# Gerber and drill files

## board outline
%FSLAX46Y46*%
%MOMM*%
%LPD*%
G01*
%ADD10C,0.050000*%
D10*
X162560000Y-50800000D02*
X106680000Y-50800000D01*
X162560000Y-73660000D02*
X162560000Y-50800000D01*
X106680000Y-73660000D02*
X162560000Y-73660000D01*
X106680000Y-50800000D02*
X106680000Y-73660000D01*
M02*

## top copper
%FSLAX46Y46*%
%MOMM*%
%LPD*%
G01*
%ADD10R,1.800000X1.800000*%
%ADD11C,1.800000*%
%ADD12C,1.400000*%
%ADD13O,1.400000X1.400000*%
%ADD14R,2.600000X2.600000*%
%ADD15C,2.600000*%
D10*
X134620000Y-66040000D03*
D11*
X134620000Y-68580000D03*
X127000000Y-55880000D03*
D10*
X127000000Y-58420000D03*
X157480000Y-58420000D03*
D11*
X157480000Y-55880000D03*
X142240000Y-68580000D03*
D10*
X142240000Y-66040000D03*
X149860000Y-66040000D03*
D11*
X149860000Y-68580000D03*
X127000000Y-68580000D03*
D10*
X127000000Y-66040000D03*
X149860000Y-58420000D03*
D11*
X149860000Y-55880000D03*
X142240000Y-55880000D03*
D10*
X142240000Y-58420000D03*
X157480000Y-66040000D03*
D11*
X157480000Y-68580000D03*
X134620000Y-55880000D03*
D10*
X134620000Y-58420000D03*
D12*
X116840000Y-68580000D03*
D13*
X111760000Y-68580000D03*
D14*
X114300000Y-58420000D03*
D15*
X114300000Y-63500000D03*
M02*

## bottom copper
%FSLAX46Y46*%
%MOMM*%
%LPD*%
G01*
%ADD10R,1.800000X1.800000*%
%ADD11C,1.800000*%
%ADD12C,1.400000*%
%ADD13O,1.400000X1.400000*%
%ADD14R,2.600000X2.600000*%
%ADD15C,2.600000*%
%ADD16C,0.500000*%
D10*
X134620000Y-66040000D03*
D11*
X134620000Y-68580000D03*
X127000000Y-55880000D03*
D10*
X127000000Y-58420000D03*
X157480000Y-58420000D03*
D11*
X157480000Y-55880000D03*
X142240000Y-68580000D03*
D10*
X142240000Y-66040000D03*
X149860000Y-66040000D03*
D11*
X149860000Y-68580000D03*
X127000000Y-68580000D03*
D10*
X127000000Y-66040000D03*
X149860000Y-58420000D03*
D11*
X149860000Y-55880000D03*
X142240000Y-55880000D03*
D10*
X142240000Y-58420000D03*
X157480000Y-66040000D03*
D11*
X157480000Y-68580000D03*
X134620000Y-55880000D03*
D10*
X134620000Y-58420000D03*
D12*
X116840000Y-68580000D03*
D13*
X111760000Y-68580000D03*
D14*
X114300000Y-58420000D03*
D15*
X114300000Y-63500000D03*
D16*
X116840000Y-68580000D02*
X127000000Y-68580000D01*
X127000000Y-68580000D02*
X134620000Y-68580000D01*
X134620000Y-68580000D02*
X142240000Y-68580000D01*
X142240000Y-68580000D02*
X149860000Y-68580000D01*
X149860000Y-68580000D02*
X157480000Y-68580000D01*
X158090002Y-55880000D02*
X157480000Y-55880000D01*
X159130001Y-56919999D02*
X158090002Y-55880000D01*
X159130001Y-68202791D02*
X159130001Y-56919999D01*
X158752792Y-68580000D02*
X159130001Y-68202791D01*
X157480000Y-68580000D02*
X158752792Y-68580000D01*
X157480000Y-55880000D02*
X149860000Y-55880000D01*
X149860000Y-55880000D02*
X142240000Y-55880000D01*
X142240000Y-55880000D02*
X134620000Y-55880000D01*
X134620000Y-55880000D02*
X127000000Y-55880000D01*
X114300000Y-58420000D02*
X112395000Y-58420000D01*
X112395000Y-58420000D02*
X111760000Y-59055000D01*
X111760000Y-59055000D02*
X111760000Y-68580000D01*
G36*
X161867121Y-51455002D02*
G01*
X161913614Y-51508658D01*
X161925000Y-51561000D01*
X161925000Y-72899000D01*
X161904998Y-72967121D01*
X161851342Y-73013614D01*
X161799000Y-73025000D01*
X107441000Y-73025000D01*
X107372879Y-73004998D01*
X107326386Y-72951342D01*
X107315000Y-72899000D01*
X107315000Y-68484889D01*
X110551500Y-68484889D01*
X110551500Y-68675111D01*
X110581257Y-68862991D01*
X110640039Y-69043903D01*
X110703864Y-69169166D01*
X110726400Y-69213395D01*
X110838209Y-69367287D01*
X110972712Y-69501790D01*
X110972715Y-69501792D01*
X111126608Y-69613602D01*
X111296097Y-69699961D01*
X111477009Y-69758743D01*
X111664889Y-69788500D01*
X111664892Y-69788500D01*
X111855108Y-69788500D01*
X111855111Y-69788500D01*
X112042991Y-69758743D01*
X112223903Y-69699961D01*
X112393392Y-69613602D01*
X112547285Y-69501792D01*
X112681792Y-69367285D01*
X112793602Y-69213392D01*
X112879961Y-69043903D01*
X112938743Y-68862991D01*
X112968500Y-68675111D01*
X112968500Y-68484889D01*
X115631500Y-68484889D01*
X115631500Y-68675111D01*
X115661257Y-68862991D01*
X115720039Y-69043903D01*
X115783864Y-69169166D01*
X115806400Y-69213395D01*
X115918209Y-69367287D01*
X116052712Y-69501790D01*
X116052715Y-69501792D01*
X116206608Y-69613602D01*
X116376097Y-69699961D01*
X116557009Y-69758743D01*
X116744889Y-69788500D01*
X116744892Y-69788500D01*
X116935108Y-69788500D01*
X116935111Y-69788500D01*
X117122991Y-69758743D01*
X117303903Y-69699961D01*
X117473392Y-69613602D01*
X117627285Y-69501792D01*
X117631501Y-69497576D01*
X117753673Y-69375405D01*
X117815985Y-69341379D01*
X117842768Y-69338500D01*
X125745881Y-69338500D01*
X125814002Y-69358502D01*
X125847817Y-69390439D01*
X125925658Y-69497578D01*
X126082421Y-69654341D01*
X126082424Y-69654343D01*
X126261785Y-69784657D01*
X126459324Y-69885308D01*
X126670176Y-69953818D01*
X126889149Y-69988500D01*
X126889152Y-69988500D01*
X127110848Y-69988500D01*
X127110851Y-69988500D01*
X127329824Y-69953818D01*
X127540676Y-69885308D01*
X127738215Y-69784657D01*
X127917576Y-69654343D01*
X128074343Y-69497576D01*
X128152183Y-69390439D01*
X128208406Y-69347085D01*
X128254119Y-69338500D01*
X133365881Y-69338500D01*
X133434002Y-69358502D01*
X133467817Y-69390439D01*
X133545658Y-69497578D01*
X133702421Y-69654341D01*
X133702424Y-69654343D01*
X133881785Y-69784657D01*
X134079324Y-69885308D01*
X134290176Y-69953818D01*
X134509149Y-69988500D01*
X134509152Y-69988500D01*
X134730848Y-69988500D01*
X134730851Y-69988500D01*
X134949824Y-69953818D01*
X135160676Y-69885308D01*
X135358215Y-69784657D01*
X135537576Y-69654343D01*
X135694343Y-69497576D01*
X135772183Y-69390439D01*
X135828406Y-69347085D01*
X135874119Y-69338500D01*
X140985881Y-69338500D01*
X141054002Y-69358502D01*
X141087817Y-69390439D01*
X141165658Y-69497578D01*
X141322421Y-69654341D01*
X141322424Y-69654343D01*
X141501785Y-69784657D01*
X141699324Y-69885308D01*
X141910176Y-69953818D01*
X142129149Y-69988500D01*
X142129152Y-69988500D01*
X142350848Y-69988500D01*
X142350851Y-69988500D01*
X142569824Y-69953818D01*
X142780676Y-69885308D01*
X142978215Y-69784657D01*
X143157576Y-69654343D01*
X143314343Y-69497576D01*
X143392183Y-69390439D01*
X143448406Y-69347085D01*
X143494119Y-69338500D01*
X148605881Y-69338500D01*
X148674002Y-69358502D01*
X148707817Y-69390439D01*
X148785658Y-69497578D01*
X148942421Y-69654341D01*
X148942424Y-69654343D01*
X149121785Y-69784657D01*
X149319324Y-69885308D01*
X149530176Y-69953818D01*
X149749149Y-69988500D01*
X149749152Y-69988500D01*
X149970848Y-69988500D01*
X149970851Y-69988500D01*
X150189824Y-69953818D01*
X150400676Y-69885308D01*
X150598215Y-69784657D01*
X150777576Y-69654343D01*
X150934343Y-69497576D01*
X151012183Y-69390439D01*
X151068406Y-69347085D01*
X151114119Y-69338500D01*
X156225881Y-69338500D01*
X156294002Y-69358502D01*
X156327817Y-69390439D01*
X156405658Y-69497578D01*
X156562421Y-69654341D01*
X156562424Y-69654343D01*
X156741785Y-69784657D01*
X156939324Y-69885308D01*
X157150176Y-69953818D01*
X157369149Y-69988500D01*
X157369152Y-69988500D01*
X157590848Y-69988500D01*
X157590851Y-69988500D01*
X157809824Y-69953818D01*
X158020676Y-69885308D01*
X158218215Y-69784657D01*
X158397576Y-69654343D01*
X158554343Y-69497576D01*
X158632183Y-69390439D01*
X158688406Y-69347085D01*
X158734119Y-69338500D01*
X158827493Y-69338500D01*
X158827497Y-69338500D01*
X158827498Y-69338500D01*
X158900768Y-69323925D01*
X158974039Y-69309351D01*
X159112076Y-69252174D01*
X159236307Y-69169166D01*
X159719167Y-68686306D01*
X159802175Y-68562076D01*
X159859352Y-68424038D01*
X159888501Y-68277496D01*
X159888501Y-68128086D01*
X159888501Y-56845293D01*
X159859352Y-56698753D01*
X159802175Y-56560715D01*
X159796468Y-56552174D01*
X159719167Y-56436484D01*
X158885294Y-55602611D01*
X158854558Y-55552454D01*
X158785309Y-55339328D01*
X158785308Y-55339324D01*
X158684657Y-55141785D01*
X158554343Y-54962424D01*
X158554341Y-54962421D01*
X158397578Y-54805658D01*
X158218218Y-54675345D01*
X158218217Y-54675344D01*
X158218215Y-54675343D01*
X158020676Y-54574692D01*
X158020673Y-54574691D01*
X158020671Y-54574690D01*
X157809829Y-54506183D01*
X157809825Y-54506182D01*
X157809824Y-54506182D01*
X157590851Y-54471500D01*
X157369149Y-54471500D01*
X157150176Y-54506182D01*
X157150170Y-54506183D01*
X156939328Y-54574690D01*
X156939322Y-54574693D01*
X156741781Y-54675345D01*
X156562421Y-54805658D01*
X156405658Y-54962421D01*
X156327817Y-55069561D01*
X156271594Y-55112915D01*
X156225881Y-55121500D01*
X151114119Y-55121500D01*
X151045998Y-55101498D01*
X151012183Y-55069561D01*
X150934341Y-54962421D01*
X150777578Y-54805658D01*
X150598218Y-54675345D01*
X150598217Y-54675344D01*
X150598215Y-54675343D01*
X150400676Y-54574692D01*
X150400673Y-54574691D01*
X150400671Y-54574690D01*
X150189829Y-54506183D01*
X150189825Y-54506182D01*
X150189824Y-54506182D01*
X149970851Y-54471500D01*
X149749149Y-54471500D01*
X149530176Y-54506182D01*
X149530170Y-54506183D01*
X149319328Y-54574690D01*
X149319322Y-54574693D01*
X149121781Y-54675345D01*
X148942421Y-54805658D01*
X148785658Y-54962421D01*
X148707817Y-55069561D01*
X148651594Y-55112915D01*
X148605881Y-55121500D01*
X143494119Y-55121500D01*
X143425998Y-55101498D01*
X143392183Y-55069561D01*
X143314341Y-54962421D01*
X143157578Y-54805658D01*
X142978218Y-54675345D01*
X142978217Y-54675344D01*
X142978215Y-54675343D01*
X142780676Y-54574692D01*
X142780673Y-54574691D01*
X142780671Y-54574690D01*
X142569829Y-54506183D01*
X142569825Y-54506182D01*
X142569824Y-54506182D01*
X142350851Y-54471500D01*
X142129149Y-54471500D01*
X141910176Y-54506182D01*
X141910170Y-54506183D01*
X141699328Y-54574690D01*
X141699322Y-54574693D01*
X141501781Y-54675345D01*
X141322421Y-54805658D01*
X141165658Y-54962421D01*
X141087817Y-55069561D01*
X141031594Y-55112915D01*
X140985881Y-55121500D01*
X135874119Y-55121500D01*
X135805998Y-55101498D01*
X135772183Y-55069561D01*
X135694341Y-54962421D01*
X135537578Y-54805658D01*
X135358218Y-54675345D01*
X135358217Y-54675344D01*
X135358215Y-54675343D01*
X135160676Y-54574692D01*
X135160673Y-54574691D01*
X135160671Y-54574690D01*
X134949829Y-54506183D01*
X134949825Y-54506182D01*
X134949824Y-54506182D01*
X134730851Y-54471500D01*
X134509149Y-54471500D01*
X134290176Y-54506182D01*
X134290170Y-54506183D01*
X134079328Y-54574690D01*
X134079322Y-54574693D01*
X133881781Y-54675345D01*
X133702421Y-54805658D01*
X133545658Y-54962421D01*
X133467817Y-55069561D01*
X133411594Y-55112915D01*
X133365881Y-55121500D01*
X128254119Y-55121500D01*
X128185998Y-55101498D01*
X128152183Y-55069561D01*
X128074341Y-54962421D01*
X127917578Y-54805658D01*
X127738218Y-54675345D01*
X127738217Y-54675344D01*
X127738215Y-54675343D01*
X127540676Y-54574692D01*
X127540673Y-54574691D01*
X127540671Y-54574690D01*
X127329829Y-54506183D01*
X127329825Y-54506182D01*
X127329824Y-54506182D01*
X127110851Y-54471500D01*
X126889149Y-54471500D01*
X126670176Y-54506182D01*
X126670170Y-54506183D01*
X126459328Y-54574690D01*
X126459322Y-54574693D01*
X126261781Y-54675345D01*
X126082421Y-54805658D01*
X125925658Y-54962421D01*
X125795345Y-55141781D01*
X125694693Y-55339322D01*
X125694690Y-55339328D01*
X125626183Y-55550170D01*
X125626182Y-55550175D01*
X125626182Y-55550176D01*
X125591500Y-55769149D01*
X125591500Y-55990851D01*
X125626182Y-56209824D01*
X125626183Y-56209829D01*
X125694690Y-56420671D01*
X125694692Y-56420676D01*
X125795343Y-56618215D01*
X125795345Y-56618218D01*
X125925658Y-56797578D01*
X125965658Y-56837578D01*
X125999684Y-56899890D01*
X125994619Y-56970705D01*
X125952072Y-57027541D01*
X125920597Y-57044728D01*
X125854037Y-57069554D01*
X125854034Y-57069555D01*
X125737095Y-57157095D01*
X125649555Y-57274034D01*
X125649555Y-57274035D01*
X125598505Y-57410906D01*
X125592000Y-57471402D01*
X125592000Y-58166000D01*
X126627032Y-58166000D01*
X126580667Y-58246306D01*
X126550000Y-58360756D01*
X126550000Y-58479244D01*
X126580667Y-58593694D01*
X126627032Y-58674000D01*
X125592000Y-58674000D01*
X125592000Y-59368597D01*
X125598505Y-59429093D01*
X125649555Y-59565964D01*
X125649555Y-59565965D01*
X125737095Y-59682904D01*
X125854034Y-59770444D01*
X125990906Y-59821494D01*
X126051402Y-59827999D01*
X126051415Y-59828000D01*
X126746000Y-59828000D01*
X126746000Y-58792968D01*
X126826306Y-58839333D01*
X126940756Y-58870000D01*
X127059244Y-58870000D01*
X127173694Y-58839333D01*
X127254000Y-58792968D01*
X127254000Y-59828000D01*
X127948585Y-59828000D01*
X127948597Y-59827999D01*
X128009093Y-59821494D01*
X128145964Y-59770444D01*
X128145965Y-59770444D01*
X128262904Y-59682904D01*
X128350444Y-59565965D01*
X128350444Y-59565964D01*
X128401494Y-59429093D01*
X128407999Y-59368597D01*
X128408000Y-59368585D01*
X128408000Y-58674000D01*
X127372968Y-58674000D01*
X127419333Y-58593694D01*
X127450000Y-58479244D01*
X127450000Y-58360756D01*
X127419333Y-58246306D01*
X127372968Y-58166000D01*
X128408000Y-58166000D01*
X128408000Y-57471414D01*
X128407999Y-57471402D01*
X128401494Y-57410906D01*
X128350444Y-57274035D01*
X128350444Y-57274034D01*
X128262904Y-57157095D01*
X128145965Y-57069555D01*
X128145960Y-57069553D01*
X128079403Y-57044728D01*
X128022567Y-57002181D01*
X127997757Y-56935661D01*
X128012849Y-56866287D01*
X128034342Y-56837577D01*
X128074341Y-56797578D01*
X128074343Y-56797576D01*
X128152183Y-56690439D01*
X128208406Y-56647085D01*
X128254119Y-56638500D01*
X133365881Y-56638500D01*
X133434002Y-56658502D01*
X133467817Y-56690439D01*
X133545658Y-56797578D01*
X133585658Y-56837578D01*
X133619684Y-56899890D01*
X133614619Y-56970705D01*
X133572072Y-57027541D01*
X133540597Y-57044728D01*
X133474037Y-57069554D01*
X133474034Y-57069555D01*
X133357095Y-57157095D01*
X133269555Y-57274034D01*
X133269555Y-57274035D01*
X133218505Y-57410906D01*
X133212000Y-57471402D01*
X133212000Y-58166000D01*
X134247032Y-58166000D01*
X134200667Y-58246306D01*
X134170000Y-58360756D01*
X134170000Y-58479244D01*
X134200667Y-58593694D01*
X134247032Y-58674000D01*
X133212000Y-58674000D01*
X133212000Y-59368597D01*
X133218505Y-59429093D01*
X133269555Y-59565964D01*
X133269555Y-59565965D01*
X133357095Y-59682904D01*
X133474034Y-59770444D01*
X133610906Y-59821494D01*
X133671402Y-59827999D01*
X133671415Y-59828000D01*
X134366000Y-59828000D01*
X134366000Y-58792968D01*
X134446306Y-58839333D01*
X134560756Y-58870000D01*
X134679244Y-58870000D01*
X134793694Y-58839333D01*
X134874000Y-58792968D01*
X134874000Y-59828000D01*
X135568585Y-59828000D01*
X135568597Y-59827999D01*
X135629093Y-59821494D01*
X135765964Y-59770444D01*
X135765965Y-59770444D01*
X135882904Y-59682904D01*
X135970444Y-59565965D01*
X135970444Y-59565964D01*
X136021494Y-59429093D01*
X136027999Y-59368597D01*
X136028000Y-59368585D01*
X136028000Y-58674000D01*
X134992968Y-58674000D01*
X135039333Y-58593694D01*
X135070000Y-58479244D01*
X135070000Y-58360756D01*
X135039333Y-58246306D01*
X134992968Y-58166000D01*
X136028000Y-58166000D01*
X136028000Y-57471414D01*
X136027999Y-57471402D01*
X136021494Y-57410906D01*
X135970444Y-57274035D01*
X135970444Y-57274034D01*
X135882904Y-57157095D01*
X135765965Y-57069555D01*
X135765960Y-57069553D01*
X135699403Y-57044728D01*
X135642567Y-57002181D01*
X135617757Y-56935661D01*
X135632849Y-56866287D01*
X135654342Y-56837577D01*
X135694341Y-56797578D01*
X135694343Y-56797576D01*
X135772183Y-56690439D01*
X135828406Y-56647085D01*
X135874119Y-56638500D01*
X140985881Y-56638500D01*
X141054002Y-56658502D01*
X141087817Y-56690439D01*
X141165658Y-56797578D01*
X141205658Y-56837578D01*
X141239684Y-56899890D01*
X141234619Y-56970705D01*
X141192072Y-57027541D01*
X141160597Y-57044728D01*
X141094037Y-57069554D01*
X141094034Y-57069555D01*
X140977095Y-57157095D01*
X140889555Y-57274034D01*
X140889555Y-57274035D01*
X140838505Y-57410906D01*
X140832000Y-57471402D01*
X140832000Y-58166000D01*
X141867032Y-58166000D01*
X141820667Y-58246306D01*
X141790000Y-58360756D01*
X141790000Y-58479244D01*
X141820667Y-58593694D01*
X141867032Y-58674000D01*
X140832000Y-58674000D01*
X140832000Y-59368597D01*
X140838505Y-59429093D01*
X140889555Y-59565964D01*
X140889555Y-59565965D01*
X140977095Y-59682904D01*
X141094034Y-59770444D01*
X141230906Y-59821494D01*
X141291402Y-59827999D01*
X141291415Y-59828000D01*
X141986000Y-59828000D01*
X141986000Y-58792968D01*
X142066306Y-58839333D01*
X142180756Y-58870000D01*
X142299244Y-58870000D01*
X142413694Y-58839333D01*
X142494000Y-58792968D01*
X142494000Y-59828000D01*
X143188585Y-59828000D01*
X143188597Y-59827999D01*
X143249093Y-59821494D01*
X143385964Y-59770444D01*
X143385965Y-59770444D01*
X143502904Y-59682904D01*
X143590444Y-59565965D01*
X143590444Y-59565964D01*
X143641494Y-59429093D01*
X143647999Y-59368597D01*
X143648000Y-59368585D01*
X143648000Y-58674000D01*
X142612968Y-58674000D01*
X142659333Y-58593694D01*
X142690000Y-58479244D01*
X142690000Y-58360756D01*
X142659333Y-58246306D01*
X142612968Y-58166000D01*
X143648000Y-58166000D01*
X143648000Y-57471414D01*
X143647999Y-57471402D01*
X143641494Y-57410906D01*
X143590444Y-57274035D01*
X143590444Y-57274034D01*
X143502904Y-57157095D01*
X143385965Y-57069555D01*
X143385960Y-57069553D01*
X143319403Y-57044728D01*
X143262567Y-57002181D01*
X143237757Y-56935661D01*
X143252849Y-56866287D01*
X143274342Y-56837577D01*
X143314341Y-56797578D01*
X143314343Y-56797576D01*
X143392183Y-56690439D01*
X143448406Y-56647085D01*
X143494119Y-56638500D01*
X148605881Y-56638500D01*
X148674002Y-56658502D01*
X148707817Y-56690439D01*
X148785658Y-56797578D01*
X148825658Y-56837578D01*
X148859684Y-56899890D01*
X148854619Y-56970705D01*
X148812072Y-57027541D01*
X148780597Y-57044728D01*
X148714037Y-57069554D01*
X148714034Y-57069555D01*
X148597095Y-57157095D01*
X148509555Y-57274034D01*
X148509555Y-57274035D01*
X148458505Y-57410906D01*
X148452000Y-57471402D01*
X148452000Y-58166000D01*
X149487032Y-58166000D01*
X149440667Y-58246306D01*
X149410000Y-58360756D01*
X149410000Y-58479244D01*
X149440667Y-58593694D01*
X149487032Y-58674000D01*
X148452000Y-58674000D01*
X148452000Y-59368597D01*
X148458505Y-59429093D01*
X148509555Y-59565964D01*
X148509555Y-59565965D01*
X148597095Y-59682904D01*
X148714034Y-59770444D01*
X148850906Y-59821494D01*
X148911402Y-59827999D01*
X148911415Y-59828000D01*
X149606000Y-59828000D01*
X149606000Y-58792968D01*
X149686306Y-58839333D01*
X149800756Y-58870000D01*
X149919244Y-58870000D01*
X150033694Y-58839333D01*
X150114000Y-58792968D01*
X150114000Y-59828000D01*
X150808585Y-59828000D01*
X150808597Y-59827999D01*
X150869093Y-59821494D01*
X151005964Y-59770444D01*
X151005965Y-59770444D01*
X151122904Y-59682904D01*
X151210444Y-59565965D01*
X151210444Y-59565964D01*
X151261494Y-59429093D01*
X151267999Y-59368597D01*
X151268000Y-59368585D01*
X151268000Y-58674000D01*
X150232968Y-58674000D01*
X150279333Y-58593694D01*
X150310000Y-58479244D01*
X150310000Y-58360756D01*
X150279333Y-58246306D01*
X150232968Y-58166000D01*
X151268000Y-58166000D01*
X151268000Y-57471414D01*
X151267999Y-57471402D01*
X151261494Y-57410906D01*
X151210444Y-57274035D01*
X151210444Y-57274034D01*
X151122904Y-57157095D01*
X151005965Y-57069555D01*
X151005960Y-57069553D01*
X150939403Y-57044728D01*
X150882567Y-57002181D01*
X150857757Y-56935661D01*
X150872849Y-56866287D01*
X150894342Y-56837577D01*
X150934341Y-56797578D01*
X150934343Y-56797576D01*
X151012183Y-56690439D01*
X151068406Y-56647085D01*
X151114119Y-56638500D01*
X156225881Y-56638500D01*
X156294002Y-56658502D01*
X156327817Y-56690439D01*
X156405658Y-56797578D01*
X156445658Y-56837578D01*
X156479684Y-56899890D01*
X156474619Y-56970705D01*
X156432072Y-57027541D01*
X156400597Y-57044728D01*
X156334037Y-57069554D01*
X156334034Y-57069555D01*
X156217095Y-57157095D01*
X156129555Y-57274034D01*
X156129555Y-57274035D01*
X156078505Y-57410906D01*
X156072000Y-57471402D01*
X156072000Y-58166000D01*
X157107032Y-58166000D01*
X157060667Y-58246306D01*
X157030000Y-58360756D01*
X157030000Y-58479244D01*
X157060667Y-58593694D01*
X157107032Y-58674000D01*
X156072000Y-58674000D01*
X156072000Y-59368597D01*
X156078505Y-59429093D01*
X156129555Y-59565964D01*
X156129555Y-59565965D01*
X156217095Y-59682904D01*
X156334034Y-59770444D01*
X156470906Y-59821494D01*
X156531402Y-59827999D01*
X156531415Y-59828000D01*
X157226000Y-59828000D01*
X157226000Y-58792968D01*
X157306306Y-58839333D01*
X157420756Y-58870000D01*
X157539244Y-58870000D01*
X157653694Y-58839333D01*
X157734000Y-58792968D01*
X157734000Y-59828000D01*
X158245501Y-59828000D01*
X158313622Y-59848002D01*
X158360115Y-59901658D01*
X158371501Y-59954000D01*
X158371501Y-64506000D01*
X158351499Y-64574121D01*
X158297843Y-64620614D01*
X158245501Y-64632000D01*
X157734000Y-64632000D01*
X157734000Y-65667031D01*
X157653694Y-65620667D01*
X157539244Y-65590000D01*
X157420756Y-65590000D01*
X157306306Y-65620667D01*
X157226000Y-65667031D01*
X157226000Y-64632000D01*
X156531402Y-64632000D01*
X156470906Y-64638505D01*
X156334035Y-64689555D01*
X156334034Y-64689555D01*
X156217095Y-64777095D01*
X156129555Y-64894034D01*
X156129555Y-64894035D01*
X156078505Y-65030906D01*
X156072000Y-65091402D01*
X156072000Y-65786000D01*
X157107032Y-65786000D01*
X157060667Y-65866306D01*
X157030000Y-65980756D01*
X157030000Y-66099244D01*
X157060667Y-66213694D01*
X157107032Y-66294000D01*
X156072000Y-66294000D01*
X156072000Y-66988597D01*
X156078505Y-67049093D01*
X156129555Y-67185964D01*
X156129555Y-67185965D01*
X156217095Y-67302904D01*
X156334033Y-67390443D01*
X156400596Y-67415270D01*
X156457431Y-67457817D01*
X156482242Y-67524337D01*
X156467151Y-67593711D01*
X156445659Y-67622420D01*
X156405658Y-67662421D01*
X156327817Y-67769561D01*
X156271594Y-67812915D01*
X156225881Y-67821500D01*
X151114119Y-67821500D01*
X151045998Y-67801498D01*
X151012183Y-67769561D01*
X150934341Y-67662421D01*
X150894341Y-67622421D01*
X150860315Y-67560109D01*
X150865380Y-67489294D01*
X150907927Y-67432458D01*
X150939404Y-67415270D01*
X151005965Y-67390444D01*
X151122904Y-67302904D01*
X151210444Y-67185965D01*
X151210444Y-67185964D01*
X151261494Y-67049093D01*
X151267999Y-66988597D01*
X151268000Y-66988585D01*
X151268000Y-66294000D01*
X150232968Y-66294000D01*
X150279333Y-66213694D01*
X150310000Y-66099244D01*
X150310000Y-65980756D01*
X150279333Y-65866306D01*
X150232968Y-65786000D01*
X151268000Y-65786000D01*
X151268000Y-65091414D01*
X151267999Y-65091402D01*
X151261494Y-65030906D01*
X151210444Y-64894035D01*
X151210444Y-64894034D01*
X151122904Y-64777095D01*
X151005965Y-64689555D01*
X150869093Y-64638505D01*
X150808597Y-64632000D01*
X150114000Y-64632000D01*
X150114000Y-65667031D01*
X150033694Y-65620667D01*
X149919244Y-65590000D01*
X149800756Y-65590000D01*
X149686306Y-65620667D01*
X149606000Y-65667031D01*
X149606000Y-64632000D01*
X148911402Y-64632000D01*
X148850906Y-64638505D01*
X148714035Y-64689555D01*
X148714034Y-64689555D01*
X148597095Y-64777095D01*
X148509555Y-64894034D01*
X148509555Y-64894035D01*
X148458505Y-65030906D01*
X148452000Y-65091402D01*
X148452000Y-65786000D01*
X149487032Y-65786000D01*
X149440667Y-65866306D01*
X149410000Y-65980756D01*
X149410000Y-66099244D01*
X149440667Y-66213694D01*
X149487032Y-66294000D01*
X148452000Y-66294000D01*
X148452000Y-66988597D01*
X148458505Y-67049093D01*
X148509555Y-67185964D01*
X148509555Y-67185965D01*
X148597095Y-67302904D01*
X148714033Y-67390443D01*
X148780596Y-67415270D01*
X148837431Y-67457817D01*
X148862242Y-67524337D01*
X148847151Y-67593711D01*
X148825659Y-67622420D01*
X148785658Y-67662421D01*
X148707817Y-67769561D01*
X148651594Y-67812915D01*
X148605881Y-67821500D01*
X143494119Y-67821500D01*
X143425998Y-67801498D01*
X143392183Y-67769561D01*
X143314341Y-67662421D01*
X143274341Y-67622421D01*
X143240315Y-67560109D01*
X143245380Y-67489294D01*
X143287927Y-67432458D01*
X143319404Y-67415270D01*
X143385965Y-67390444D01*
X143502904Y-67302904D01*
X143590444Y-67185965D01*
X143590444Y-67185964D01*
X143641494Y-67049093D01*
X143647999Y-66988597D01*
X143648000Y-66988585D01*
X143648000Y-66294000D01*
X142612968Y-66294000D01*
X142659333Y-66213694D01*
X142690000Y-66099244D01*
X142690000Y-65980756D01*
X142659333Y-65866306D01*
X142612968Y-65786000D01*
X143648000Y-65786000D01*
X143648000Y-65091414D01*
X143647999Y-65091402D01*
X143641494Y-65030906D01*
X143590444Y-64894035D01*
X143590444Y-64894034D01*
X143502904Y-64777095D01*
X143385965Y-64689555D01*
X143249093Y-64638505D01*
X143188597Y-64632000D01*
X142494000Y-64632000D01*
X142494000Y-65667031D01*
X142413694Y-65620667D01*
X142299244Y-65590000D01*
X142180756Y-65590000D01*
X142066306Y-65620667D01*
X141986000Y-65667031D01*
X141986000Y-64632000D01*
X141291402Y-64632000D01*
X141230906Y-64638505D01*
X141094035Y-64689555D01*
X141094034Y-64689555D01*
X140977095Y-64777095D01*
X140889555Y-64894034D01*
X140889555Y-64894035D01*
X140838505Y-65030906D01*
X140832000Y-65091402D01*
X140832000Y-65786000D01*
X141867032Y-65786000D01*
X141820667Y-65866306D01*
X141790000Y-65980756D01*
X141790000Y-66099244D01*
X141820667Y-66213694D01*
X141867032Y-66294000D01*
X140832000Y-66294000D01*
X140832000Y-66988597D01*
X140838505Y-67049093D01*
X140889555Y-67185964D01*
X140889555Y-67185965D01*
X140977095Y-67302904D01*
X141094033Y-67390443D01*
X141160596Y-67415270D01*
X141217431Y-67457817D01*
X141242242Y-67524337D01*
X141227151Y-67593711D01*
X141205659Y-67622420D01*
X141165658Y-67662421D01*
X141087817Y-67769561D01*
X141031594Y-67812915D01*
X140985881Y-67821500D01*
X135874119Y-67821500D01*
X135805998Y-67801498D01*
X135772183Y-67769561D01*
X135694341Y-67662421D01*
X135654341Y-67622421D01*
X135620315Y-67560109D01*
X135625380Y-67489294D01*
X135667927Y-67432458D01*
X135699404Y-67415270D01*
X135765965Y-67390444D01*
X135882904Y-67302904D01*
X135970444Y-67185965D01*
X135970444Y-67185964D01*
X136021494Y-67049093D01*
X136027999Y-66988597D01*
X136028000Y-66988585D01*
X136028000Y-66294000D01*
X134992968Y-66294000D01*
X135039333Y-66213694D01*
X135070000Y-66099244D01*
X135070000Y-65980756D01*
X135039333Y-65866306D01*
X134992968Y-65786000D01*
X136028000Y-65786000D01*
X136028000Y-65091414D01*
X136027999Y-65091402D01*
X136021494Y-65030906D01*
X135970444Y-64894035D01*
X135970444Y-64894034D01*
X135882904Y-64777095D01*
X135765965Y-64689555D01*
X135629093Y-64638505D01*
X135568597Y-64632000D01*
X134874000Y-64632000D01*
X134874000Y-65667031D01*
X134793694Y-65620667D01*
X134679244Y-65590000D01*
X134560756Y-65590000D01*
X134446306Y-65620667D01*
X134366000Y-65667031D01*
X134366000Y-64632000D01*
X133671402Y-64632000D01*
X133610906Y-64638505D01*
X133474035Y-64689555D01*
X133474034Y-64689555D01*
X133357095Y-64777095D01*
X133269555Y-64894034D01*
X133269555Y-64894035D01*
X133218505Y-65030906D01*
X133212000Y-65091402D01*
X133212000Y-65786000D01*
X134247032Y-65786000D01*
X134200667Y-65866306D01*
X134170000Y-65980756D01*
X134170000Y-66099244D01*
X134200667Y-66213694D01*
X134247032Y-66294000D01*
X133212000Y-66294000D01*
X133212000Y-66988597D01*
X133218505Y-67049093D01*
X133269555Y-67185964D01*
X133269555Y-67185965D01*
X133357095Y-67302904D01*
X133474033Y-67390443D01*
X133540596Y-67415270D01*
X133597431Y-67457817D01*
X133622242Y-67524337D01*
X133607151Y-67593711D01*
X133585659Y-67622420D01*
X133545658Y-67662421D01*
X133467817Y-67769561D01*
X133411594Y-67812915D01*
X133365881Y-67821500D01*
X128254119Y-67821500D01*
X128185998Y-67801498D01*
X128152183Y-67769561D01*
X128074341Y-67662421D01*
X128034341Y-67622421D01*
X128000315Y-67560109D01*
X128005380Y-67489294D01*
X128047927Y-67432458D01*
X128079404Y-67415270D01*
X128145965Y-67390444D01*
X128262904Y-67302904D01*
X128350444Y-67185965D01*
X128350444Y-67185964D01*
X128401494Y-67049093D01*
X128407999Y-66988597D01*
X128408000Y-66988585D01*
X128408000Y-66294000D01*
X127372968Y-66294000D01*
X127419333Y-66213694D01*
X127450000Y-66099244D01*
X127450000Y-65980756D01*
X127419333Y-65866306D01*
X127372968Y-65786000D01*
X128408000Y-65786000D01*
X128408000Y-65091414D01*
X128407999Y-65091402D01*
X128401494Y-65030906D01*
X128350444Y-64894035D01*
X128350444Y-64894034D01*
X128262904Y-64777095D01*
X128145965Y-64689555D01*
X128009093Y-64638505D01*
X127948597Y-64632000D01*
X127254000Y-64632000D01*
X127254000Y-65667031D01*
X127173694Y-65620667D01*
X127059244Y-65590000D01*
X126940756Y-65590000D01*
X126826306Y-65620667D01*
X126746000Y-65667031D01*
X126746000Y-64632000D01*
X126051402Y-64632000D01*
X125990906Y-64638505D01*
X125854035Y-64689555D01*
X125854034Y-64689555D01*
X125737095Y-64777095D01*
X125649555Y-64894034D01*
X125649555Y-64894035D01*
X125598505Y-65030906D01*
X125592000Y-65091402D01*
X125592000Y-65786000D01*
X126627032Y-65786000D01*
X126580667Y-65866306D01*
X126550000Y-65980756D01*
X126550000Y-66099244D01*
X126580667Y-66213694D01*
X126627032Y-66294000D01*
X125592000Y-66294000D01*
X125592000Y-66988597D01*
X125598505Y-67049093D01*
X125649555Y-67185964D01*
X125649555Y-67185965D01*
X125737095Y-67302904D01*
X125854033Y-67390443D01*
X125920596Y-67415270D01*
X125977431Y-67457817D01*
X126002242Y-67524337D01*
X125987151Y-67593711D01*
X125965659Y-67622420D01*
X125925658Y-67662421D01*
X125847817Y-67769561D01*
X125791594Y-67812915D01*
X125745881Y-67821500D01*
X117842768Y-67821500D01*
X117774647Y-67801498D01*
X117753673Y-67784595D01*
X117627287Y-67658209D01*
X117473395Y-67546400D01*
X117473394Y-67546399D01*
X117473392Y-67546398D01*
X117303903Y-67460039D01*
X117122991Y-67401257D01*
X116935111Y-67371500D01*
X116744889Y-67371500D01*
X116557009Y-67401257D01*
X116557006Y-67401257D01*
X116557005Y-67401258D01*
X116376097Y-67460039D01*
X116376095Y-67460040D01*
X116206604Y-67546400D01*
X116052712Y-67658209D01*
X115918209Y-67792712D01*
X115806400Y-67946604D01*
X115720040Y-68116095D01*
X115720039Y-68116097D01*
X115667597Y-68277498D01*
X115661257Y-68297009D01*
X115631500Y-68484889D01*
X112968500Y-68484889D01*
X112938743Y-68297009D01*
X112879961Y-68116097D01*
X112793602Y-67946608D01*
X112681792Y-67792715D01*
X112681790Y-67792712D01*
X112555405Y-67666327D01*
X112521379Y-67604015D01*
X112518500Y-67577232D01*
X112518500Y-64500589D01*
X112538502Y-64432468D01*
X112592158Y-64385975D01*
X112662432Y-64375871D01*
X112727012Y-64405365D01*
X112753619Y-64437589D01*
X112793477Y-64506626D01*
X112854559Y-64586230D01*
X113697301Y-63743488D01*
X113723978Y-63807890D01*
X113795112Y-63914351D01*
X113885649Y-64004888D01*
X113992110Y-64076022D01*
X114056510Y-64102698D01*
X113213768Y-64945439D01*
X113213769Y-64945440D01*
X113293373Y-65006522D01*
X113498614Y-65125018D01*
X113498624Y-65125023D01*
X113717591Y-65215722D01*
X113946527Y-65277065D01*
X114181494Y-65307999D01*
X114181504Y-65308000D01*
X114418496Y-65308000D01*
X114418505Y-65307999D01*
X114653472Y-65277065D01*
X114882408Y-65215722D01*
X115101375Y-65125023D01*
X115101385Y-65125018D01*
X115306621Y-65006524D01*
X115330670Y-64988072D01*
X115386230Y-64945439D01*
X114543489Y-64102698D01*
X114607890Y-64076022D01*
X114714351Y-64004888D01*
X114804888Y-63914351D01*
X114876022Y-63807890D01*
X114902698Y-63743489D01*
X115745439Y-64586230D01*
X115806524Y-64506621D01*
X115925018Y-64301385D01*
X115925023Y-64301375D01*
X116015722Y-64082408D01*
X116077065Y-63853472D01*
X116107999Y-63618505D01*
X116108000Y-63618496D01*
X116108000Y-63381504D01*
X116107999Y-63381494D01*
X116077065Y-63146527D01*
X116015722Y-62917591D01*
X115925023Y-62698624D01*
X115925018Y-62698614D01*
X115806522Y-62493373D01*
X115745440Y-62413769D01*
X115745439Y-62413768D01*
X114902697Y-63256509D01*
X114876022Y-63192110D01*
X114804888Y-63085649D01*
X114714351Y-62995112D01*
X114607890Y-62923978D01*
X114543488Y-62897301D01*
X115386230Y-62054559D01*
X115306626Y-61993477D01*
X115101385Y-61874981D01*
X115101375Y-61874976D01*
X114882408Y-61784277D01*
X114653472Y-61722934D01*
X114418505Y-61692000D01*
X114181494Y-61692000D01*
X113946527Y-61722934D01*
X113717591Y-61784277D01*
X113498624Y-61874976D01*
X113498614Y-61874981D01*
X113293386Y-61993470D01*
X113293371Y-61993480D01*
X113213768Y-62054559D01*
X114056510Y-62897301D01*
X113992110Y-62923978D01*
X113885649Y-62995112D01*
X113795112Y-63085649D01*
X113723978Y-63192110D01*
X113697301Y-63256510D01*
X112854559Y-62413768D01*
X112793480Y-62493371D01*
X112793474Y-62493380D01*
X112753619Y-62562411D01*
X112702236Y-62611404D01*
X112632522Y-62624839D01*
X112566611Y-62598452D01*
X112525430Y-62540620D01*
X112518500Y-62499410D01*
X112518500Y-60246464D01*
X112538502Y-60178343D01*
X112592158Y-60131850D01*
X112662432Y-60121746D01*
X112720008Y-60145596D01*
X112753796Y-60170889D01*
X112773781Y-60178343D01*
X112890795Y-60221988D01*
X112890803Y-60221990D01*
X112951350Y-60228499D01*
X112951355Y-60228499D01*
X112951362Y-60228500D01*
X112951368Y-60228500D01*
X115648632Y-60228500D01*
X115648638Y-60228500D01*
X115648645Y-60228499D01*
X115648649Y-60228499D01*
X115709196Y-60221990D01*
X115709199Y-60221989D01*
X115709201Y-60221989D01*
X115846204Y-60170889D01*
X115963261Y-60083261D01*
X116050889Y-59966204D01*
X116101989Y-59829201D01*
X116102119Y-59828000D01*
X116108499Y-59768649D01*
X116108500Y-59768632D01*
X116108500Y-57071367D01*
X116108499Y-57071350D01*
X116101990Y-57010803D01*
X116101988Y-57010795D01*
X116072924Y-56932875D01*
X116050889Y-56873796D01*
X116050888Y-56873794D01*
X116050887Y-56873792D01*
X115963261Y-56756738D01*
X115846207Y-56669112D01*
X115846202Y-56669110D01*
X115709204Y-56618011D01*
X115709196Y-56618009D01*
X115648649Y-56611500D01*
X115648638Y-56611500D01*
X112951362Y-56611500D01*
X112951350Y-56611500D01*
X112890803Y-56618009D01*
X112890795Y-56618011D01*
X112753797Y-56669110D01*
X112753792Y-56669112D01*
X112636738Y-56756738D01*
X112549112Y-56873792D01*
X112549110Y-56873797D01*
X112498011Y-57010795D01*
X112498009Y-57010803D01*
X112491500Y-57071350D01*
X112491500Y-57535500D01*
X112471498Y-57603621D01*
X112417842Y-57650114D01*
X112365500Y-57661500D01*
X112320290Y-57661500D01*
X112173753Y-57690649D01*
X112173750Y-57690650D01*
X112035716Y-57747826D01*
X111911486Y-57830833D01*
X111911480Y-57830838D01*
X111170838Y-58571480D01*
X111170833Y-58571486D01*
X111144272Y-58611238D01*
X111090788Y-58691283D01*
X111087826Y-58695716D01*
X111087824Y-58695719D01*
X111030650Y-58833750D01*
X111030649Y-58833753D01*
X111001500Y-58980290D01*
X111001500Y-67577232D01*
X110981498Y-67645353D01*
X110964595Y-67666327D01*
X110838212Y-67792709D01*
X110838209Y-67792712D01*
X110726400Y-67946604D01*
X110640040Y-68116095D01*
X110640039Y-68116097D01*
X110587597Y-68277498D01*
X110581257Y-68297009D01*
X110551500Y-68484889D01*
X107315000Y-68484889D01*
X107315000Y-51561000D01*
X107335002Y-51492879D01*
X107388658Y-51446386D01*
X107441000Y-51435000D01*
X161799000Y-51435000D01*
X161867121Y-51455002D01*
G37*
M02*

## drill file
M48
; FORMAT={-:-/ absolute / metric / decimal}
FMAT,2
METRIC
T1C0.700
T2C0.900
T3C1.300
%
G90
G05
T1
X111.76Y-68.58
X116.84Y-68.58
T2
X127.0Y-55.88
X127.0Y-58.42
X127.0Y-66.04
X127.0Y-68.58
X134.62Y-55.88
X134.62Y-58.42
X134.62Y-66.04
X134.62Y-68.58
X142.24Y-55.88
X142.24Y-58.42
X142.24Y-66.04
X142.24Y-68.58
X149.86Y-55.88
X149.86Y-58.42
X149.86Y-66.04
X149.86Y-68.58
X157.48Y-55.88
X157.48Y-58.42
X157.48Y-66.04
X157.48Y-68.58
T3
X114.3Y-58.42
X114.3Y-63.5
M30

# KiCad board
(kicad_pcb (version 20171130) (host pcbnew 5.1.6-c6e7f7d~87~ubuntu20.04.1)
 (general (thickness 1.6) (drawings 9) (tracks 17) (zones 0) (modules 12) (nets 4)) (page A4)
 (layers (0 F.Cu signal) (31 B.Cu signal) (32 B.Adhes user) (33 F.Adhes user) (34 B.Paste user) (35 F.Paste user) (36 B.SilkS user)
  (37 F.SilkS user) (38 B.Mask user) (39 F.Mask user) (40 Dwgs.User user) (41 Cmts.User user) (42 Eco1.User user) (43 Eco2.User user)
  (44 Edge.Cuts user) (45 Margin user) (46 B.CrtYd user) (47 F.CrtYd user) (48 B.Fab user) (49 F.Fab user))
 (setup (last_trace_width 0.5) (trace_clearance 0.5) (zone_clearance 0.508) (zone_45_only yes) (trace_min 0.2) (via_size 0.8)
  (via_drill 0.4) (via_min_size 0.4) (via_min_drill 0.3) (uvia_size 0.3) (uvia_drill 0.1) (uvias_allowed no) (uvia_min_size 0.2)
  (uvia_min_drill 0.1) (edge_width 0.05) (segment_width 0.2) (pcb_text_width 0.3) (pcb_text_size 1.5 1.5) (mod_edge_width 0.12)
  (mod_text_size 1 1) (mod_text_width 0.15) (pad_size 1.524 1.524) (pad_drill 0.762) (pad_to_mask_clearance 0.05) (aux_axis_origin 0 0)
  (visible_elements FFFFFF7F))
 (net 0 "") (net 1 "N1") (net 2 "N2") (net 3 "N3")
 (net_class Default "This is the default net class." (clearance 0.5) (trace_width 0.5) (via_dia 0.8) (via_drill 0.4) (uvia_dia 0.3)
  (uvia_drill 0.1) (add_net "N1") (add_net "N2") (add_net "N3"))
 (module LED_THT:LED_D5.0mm (layer F.Cu) (at 134.62 66.04 270)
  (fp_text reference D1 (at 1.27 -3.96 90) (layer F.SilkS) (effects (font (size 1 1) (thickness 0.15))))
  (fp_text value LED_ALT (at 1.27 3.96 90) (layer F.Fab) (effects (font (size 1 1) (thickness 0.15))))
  (pad 1 thru_hole rect (at 0 0 270) (size 1.8 1.8) (drill 0.9) (layers *.Cu *.Mask) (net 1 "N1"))
  (pad 2 thru_hole circle (at 2.54 0 270) (size 1.8 1.8) (drill 0.9) (layers *.Cu *.Mask) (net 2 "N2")))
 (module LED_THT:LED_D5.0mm (layer F.Cu) (at 127 58.42 90)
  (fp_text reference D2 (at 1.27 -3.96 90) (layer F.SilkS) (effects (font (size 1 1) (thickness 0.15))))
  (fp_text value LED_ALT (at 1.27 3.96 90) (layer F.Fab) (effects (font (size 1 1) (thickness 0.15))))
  (pad 2 thru_hole circle (at 2.54 0 90) (size 1.8 1.8) (drill 0.9) (layers *.Cu *.Mask) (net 2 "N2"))
  (pad 1 thru_hole rect (at 0 0 90) (size 1.8 1.8) (drill 0.9) (layers *.Cu *.Mask) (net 1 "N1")))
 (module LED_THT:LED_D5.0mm (layer F.Cu) (at 157.48 58.42 90)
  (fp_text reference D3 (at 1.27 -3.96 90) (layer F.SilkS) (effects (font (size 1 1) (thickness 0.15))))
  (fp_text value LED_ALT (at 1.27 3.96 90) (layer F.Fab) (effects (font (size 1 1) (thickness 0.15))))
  (pad 1 thru_hole rect (at 0 0 90) (size 1.8 1.8) (drill 0.9) (layers *.Cu *.Mask) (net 1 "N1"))
  (pad 2 thru_hole circle (at 2.54 0 90) (size 1.8 1.8) (drill 0.9) (layers *.Cu *.Mask) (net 2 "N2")))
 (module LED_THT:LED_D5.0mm (layer F.Cu) (at 142.24 66.04 270)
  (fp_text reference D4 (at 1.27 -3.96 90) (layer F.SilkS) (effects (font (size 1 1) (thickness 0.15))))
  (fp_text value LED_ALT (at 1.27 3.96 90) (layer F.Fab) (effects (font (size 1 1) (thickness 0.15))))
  (pad 2 thru_hole circle (at 2.54 0 270) (size 1.8 1.8) (drill 0.9) (layers *.Cu *.Mask) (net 2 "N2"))
  (pad 1 thru_hole rect (at 0 0 270) (size 1.8 1.8) (drill 0.9) (layers *.Cu *.Mask) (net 1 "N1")))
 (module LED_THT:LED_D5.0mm (layer F.Cu) (at 149.86 66.04 270)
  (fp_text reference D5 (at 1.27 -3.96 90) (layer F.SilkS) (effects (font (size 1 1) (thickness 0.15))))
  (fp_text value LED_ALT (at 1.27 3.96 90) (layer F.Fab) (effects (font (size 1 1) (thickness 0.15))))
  (pad 1 thru_hole rect (at 0 0 270) (size 1.8 1.8) (drill 0.9) (layers *.Cu *.Mask) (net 1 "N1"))
  (pad 2 thru_hole circle (at 2.54 0 270) (size 1.8 1.8) (drill 0.9) (layers *.Cu *.Mask) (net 2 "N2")))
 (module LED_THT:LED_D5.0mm (layer F.Cu) (at 127 66.04 270)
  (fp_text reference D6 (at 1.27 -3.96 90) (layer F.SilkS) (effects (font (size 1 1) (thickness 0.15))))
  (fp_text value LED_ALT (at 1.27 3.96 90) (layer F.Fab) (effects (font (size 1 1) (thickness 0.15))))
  (pad 2 thru_hole circle (at 2.54 0 270) (size 1.8 1.8) (drill 0.9) (layers *.Cu *.Mask) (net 2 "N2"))
  (pad 1 thru_hole rect (at 0 0 270) (size 1.8 1.8) (drill 0.9) (layers *.Cu *.Mask) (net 1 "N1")))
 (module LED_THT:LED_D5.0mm (layer F.Cu) (at 149.86 58.42 90)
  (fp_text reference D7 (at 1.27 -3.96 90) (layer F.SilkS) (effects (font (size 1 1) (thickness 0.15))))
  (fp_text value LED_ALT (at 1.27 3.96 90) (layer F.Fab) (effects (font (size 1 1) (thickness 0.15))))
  (pad 1 thru_hole rect (at 0 0 90) (size 1.8 1.8) (drill 0.9) (layers *.Cu *.Mask) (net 1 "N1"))
  (pad 2 thru_hole circle (at 2.54 0 90) (size 1.8 1.8) (drill 0.9) (layers *.Cu *.Mask) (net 2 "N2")))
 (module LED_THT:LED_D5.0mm (layer F.Cu) (at 142.24 58.42 90)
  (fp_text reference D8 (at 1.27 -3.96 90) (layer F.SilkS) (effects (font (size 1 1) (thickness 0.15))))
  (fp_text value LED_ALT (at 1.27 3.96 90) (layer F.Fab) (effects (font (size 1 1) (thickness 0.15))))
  (pad 2 thru_hole circle (at 2.54 0 90) (size 1.8 1.8) (drill 0.9) (layers *.Cu *.Mask) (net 2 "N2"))
  (pad 1 thru_hole rect (at 0 0 90) (size 1.8 1.8) (drill 0.9) (layers *.Cu *.Mask) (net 1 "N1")))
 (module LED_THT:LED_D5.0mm (layer F.Cu) (at 157.48 66.04 270)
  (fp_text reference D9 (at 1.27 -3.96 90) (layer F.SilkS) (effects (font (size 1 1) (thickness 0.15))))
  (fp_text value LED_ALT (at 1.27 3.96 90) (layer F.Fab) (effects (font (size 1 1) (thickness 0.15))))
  (pad 1 thru_hole rect (at 0 0 270) (size 1.8 1.8) (drill 0.9) (layers *.Cu *.Mask) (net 1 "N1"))
  (pad 2 thru_hole circle (at 2.54 0 270) (size 1.8 1.8) (drill 0.9) (layers *.Cu *.Mask) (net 2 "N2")))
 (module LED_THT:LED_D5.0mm (layer F.Cu) (at 134.62 58.42 90)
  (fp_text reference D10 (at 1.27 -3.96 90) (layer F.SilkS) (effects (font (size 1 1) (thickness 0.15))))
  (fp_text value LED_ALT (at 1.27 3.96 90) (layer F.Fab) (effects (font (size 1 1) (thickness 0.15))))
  (pad 2 thru_hole circle (at 2.54 0 90) (size 1.8 1.8) (drill 0.9) (layers *.Cu *.Mask) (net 2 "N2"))
  (pad 1 thru_hole rect (at 0 0 90) (size 1.8 1.8) (drill 0.9) (layers *.Cu *.Mask) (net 1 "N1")))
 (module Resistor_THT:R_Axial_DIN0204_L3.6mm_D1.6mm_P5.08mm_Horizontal (layer F.Cu) (at 116.84 68.58 180)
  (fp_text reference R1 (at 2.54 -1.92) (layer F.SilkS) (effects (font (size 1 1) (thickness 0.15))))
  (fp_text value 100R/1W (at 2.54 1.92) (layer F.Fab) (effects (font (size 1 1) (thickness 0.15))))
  (pad 1 thru_hole circle (at 0 0 180) (size 1.4 1.4) (drill 0.7) (layers *.Cu *.Mask) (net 2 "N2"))
  (pad 2 thru_hole oval (at 5.08 0 180) (size 1.4 1.4) (drill 0.7) (layers *.Cu *.Mask) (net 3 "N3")))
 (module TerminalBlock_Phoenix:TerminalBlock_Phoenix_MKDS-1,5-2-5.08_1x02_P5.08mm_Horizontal (layer F.Cu) (at 114.3 58.42 270)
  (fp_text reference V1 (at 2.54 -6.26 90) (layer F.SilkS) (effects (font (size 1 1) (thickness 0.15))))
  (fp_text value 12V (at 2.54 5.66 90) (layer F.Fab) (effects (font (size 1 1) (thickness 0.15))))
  (pad 1 thru_hole rect (at 0 0 270) (size 2.6 2.6) (drill 1.3) (layers *.Cu *.Mask) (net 3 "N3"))
  (pad 2 thru_hole circle (at 5.08 0 270) (size 2.6 2.6) (drill 1.3) (layers *.Cu *.Mask) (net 1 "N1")))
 (gr_line (start 162.56 50.8) (end 106.68 50.8) (layer Edge.Cuts) (width 0.05))
 (gr_line (start 162.56 73.66) (end 162.56 50.8) (layer Edge.Cuts) (width 0.05))
 (gr_line (start 106.68 73.66) (end 162.56 73.66) (layer Edge.Cuts) (width 0.05))
 (gr_line (start 106.68 50.8) (end 106.68 73.66) (layer Edge.Cuts) (width 0.05))
 (segment (start 116.84 68.58) (end 127 68.58) (width 0.5) (layer B.Cu) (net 2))
 (segment (start 127 68.58) (end 134.62 68.58) (width 0.5) (layer B.Cu) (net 2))
 (segment (start 134.62 68.58) (end 142.24 68.58) (width 0.5) (layer B.Cu) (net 2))
 (segment (start 142.24 68.58) (end 149.86 68.58) (width 0.5) (layer B.Cu) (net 2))
 (segment (start 149.86 68.58) (end 157.48 68.58) (width 0.5) (layer B.Cu) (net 2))
 (segment (start 158.090002 55.88) (end 157.48 55.88) (width 0.5) (layer B.Cu) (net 2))
 (segment (start 159.130001 56.919999) (end 158.090002 55.88) (width 0.5) (layer B.Cu) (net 2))
 (segment (start 159.130001 68.202791) (end 159.130001 56.919999) (width 0.5) (layer B.Cu) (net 2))
 (segment (start 158.752792 68.58) (end 159.130001 68.202791) (width 0.5) (layer B.Cu) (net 2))
 (segment (start 157.48 68.58) (end 158.752792 68.58) (width 0.5) (layer B.Cu) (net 2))
 (segment (start 157.48 55.88) (end 149.86 55.88) (width 0.5) (layer B.Cu) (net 2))
 (segment (start 149.86 55.88) (end 142.24 55.88) (width 0.5) (layer B.Cu) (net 2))
 (segment (start 142.24 55.88) (end 134.62 55.88) (width 0.5) (layer B.Cu) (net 2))
 (segment (start 134.62 55.88) (end 127 55.88) (width 0.5) (layer B.Cu) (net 2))
 (segment (start 114.3 58.42) (end 112.395 58.42) (width 0.5) (layer B.Cu) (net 3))
 (segment (start 112.395 58.42) (end 111.76 59.055) (width 0.5) (layer B.Cu) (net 3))
 (segment (start 111.76 59.055) (end 111.76 68.58) (width 0.5) (layer B.Cu) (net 3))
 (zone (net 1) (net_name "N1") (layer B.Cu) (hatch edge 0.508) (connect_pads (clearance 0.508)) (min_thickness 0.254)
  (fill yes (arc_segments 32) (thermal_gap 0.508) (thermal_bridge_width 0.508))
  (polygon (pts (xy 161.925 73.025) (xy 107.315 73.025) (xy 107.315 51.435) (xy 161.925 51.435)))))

